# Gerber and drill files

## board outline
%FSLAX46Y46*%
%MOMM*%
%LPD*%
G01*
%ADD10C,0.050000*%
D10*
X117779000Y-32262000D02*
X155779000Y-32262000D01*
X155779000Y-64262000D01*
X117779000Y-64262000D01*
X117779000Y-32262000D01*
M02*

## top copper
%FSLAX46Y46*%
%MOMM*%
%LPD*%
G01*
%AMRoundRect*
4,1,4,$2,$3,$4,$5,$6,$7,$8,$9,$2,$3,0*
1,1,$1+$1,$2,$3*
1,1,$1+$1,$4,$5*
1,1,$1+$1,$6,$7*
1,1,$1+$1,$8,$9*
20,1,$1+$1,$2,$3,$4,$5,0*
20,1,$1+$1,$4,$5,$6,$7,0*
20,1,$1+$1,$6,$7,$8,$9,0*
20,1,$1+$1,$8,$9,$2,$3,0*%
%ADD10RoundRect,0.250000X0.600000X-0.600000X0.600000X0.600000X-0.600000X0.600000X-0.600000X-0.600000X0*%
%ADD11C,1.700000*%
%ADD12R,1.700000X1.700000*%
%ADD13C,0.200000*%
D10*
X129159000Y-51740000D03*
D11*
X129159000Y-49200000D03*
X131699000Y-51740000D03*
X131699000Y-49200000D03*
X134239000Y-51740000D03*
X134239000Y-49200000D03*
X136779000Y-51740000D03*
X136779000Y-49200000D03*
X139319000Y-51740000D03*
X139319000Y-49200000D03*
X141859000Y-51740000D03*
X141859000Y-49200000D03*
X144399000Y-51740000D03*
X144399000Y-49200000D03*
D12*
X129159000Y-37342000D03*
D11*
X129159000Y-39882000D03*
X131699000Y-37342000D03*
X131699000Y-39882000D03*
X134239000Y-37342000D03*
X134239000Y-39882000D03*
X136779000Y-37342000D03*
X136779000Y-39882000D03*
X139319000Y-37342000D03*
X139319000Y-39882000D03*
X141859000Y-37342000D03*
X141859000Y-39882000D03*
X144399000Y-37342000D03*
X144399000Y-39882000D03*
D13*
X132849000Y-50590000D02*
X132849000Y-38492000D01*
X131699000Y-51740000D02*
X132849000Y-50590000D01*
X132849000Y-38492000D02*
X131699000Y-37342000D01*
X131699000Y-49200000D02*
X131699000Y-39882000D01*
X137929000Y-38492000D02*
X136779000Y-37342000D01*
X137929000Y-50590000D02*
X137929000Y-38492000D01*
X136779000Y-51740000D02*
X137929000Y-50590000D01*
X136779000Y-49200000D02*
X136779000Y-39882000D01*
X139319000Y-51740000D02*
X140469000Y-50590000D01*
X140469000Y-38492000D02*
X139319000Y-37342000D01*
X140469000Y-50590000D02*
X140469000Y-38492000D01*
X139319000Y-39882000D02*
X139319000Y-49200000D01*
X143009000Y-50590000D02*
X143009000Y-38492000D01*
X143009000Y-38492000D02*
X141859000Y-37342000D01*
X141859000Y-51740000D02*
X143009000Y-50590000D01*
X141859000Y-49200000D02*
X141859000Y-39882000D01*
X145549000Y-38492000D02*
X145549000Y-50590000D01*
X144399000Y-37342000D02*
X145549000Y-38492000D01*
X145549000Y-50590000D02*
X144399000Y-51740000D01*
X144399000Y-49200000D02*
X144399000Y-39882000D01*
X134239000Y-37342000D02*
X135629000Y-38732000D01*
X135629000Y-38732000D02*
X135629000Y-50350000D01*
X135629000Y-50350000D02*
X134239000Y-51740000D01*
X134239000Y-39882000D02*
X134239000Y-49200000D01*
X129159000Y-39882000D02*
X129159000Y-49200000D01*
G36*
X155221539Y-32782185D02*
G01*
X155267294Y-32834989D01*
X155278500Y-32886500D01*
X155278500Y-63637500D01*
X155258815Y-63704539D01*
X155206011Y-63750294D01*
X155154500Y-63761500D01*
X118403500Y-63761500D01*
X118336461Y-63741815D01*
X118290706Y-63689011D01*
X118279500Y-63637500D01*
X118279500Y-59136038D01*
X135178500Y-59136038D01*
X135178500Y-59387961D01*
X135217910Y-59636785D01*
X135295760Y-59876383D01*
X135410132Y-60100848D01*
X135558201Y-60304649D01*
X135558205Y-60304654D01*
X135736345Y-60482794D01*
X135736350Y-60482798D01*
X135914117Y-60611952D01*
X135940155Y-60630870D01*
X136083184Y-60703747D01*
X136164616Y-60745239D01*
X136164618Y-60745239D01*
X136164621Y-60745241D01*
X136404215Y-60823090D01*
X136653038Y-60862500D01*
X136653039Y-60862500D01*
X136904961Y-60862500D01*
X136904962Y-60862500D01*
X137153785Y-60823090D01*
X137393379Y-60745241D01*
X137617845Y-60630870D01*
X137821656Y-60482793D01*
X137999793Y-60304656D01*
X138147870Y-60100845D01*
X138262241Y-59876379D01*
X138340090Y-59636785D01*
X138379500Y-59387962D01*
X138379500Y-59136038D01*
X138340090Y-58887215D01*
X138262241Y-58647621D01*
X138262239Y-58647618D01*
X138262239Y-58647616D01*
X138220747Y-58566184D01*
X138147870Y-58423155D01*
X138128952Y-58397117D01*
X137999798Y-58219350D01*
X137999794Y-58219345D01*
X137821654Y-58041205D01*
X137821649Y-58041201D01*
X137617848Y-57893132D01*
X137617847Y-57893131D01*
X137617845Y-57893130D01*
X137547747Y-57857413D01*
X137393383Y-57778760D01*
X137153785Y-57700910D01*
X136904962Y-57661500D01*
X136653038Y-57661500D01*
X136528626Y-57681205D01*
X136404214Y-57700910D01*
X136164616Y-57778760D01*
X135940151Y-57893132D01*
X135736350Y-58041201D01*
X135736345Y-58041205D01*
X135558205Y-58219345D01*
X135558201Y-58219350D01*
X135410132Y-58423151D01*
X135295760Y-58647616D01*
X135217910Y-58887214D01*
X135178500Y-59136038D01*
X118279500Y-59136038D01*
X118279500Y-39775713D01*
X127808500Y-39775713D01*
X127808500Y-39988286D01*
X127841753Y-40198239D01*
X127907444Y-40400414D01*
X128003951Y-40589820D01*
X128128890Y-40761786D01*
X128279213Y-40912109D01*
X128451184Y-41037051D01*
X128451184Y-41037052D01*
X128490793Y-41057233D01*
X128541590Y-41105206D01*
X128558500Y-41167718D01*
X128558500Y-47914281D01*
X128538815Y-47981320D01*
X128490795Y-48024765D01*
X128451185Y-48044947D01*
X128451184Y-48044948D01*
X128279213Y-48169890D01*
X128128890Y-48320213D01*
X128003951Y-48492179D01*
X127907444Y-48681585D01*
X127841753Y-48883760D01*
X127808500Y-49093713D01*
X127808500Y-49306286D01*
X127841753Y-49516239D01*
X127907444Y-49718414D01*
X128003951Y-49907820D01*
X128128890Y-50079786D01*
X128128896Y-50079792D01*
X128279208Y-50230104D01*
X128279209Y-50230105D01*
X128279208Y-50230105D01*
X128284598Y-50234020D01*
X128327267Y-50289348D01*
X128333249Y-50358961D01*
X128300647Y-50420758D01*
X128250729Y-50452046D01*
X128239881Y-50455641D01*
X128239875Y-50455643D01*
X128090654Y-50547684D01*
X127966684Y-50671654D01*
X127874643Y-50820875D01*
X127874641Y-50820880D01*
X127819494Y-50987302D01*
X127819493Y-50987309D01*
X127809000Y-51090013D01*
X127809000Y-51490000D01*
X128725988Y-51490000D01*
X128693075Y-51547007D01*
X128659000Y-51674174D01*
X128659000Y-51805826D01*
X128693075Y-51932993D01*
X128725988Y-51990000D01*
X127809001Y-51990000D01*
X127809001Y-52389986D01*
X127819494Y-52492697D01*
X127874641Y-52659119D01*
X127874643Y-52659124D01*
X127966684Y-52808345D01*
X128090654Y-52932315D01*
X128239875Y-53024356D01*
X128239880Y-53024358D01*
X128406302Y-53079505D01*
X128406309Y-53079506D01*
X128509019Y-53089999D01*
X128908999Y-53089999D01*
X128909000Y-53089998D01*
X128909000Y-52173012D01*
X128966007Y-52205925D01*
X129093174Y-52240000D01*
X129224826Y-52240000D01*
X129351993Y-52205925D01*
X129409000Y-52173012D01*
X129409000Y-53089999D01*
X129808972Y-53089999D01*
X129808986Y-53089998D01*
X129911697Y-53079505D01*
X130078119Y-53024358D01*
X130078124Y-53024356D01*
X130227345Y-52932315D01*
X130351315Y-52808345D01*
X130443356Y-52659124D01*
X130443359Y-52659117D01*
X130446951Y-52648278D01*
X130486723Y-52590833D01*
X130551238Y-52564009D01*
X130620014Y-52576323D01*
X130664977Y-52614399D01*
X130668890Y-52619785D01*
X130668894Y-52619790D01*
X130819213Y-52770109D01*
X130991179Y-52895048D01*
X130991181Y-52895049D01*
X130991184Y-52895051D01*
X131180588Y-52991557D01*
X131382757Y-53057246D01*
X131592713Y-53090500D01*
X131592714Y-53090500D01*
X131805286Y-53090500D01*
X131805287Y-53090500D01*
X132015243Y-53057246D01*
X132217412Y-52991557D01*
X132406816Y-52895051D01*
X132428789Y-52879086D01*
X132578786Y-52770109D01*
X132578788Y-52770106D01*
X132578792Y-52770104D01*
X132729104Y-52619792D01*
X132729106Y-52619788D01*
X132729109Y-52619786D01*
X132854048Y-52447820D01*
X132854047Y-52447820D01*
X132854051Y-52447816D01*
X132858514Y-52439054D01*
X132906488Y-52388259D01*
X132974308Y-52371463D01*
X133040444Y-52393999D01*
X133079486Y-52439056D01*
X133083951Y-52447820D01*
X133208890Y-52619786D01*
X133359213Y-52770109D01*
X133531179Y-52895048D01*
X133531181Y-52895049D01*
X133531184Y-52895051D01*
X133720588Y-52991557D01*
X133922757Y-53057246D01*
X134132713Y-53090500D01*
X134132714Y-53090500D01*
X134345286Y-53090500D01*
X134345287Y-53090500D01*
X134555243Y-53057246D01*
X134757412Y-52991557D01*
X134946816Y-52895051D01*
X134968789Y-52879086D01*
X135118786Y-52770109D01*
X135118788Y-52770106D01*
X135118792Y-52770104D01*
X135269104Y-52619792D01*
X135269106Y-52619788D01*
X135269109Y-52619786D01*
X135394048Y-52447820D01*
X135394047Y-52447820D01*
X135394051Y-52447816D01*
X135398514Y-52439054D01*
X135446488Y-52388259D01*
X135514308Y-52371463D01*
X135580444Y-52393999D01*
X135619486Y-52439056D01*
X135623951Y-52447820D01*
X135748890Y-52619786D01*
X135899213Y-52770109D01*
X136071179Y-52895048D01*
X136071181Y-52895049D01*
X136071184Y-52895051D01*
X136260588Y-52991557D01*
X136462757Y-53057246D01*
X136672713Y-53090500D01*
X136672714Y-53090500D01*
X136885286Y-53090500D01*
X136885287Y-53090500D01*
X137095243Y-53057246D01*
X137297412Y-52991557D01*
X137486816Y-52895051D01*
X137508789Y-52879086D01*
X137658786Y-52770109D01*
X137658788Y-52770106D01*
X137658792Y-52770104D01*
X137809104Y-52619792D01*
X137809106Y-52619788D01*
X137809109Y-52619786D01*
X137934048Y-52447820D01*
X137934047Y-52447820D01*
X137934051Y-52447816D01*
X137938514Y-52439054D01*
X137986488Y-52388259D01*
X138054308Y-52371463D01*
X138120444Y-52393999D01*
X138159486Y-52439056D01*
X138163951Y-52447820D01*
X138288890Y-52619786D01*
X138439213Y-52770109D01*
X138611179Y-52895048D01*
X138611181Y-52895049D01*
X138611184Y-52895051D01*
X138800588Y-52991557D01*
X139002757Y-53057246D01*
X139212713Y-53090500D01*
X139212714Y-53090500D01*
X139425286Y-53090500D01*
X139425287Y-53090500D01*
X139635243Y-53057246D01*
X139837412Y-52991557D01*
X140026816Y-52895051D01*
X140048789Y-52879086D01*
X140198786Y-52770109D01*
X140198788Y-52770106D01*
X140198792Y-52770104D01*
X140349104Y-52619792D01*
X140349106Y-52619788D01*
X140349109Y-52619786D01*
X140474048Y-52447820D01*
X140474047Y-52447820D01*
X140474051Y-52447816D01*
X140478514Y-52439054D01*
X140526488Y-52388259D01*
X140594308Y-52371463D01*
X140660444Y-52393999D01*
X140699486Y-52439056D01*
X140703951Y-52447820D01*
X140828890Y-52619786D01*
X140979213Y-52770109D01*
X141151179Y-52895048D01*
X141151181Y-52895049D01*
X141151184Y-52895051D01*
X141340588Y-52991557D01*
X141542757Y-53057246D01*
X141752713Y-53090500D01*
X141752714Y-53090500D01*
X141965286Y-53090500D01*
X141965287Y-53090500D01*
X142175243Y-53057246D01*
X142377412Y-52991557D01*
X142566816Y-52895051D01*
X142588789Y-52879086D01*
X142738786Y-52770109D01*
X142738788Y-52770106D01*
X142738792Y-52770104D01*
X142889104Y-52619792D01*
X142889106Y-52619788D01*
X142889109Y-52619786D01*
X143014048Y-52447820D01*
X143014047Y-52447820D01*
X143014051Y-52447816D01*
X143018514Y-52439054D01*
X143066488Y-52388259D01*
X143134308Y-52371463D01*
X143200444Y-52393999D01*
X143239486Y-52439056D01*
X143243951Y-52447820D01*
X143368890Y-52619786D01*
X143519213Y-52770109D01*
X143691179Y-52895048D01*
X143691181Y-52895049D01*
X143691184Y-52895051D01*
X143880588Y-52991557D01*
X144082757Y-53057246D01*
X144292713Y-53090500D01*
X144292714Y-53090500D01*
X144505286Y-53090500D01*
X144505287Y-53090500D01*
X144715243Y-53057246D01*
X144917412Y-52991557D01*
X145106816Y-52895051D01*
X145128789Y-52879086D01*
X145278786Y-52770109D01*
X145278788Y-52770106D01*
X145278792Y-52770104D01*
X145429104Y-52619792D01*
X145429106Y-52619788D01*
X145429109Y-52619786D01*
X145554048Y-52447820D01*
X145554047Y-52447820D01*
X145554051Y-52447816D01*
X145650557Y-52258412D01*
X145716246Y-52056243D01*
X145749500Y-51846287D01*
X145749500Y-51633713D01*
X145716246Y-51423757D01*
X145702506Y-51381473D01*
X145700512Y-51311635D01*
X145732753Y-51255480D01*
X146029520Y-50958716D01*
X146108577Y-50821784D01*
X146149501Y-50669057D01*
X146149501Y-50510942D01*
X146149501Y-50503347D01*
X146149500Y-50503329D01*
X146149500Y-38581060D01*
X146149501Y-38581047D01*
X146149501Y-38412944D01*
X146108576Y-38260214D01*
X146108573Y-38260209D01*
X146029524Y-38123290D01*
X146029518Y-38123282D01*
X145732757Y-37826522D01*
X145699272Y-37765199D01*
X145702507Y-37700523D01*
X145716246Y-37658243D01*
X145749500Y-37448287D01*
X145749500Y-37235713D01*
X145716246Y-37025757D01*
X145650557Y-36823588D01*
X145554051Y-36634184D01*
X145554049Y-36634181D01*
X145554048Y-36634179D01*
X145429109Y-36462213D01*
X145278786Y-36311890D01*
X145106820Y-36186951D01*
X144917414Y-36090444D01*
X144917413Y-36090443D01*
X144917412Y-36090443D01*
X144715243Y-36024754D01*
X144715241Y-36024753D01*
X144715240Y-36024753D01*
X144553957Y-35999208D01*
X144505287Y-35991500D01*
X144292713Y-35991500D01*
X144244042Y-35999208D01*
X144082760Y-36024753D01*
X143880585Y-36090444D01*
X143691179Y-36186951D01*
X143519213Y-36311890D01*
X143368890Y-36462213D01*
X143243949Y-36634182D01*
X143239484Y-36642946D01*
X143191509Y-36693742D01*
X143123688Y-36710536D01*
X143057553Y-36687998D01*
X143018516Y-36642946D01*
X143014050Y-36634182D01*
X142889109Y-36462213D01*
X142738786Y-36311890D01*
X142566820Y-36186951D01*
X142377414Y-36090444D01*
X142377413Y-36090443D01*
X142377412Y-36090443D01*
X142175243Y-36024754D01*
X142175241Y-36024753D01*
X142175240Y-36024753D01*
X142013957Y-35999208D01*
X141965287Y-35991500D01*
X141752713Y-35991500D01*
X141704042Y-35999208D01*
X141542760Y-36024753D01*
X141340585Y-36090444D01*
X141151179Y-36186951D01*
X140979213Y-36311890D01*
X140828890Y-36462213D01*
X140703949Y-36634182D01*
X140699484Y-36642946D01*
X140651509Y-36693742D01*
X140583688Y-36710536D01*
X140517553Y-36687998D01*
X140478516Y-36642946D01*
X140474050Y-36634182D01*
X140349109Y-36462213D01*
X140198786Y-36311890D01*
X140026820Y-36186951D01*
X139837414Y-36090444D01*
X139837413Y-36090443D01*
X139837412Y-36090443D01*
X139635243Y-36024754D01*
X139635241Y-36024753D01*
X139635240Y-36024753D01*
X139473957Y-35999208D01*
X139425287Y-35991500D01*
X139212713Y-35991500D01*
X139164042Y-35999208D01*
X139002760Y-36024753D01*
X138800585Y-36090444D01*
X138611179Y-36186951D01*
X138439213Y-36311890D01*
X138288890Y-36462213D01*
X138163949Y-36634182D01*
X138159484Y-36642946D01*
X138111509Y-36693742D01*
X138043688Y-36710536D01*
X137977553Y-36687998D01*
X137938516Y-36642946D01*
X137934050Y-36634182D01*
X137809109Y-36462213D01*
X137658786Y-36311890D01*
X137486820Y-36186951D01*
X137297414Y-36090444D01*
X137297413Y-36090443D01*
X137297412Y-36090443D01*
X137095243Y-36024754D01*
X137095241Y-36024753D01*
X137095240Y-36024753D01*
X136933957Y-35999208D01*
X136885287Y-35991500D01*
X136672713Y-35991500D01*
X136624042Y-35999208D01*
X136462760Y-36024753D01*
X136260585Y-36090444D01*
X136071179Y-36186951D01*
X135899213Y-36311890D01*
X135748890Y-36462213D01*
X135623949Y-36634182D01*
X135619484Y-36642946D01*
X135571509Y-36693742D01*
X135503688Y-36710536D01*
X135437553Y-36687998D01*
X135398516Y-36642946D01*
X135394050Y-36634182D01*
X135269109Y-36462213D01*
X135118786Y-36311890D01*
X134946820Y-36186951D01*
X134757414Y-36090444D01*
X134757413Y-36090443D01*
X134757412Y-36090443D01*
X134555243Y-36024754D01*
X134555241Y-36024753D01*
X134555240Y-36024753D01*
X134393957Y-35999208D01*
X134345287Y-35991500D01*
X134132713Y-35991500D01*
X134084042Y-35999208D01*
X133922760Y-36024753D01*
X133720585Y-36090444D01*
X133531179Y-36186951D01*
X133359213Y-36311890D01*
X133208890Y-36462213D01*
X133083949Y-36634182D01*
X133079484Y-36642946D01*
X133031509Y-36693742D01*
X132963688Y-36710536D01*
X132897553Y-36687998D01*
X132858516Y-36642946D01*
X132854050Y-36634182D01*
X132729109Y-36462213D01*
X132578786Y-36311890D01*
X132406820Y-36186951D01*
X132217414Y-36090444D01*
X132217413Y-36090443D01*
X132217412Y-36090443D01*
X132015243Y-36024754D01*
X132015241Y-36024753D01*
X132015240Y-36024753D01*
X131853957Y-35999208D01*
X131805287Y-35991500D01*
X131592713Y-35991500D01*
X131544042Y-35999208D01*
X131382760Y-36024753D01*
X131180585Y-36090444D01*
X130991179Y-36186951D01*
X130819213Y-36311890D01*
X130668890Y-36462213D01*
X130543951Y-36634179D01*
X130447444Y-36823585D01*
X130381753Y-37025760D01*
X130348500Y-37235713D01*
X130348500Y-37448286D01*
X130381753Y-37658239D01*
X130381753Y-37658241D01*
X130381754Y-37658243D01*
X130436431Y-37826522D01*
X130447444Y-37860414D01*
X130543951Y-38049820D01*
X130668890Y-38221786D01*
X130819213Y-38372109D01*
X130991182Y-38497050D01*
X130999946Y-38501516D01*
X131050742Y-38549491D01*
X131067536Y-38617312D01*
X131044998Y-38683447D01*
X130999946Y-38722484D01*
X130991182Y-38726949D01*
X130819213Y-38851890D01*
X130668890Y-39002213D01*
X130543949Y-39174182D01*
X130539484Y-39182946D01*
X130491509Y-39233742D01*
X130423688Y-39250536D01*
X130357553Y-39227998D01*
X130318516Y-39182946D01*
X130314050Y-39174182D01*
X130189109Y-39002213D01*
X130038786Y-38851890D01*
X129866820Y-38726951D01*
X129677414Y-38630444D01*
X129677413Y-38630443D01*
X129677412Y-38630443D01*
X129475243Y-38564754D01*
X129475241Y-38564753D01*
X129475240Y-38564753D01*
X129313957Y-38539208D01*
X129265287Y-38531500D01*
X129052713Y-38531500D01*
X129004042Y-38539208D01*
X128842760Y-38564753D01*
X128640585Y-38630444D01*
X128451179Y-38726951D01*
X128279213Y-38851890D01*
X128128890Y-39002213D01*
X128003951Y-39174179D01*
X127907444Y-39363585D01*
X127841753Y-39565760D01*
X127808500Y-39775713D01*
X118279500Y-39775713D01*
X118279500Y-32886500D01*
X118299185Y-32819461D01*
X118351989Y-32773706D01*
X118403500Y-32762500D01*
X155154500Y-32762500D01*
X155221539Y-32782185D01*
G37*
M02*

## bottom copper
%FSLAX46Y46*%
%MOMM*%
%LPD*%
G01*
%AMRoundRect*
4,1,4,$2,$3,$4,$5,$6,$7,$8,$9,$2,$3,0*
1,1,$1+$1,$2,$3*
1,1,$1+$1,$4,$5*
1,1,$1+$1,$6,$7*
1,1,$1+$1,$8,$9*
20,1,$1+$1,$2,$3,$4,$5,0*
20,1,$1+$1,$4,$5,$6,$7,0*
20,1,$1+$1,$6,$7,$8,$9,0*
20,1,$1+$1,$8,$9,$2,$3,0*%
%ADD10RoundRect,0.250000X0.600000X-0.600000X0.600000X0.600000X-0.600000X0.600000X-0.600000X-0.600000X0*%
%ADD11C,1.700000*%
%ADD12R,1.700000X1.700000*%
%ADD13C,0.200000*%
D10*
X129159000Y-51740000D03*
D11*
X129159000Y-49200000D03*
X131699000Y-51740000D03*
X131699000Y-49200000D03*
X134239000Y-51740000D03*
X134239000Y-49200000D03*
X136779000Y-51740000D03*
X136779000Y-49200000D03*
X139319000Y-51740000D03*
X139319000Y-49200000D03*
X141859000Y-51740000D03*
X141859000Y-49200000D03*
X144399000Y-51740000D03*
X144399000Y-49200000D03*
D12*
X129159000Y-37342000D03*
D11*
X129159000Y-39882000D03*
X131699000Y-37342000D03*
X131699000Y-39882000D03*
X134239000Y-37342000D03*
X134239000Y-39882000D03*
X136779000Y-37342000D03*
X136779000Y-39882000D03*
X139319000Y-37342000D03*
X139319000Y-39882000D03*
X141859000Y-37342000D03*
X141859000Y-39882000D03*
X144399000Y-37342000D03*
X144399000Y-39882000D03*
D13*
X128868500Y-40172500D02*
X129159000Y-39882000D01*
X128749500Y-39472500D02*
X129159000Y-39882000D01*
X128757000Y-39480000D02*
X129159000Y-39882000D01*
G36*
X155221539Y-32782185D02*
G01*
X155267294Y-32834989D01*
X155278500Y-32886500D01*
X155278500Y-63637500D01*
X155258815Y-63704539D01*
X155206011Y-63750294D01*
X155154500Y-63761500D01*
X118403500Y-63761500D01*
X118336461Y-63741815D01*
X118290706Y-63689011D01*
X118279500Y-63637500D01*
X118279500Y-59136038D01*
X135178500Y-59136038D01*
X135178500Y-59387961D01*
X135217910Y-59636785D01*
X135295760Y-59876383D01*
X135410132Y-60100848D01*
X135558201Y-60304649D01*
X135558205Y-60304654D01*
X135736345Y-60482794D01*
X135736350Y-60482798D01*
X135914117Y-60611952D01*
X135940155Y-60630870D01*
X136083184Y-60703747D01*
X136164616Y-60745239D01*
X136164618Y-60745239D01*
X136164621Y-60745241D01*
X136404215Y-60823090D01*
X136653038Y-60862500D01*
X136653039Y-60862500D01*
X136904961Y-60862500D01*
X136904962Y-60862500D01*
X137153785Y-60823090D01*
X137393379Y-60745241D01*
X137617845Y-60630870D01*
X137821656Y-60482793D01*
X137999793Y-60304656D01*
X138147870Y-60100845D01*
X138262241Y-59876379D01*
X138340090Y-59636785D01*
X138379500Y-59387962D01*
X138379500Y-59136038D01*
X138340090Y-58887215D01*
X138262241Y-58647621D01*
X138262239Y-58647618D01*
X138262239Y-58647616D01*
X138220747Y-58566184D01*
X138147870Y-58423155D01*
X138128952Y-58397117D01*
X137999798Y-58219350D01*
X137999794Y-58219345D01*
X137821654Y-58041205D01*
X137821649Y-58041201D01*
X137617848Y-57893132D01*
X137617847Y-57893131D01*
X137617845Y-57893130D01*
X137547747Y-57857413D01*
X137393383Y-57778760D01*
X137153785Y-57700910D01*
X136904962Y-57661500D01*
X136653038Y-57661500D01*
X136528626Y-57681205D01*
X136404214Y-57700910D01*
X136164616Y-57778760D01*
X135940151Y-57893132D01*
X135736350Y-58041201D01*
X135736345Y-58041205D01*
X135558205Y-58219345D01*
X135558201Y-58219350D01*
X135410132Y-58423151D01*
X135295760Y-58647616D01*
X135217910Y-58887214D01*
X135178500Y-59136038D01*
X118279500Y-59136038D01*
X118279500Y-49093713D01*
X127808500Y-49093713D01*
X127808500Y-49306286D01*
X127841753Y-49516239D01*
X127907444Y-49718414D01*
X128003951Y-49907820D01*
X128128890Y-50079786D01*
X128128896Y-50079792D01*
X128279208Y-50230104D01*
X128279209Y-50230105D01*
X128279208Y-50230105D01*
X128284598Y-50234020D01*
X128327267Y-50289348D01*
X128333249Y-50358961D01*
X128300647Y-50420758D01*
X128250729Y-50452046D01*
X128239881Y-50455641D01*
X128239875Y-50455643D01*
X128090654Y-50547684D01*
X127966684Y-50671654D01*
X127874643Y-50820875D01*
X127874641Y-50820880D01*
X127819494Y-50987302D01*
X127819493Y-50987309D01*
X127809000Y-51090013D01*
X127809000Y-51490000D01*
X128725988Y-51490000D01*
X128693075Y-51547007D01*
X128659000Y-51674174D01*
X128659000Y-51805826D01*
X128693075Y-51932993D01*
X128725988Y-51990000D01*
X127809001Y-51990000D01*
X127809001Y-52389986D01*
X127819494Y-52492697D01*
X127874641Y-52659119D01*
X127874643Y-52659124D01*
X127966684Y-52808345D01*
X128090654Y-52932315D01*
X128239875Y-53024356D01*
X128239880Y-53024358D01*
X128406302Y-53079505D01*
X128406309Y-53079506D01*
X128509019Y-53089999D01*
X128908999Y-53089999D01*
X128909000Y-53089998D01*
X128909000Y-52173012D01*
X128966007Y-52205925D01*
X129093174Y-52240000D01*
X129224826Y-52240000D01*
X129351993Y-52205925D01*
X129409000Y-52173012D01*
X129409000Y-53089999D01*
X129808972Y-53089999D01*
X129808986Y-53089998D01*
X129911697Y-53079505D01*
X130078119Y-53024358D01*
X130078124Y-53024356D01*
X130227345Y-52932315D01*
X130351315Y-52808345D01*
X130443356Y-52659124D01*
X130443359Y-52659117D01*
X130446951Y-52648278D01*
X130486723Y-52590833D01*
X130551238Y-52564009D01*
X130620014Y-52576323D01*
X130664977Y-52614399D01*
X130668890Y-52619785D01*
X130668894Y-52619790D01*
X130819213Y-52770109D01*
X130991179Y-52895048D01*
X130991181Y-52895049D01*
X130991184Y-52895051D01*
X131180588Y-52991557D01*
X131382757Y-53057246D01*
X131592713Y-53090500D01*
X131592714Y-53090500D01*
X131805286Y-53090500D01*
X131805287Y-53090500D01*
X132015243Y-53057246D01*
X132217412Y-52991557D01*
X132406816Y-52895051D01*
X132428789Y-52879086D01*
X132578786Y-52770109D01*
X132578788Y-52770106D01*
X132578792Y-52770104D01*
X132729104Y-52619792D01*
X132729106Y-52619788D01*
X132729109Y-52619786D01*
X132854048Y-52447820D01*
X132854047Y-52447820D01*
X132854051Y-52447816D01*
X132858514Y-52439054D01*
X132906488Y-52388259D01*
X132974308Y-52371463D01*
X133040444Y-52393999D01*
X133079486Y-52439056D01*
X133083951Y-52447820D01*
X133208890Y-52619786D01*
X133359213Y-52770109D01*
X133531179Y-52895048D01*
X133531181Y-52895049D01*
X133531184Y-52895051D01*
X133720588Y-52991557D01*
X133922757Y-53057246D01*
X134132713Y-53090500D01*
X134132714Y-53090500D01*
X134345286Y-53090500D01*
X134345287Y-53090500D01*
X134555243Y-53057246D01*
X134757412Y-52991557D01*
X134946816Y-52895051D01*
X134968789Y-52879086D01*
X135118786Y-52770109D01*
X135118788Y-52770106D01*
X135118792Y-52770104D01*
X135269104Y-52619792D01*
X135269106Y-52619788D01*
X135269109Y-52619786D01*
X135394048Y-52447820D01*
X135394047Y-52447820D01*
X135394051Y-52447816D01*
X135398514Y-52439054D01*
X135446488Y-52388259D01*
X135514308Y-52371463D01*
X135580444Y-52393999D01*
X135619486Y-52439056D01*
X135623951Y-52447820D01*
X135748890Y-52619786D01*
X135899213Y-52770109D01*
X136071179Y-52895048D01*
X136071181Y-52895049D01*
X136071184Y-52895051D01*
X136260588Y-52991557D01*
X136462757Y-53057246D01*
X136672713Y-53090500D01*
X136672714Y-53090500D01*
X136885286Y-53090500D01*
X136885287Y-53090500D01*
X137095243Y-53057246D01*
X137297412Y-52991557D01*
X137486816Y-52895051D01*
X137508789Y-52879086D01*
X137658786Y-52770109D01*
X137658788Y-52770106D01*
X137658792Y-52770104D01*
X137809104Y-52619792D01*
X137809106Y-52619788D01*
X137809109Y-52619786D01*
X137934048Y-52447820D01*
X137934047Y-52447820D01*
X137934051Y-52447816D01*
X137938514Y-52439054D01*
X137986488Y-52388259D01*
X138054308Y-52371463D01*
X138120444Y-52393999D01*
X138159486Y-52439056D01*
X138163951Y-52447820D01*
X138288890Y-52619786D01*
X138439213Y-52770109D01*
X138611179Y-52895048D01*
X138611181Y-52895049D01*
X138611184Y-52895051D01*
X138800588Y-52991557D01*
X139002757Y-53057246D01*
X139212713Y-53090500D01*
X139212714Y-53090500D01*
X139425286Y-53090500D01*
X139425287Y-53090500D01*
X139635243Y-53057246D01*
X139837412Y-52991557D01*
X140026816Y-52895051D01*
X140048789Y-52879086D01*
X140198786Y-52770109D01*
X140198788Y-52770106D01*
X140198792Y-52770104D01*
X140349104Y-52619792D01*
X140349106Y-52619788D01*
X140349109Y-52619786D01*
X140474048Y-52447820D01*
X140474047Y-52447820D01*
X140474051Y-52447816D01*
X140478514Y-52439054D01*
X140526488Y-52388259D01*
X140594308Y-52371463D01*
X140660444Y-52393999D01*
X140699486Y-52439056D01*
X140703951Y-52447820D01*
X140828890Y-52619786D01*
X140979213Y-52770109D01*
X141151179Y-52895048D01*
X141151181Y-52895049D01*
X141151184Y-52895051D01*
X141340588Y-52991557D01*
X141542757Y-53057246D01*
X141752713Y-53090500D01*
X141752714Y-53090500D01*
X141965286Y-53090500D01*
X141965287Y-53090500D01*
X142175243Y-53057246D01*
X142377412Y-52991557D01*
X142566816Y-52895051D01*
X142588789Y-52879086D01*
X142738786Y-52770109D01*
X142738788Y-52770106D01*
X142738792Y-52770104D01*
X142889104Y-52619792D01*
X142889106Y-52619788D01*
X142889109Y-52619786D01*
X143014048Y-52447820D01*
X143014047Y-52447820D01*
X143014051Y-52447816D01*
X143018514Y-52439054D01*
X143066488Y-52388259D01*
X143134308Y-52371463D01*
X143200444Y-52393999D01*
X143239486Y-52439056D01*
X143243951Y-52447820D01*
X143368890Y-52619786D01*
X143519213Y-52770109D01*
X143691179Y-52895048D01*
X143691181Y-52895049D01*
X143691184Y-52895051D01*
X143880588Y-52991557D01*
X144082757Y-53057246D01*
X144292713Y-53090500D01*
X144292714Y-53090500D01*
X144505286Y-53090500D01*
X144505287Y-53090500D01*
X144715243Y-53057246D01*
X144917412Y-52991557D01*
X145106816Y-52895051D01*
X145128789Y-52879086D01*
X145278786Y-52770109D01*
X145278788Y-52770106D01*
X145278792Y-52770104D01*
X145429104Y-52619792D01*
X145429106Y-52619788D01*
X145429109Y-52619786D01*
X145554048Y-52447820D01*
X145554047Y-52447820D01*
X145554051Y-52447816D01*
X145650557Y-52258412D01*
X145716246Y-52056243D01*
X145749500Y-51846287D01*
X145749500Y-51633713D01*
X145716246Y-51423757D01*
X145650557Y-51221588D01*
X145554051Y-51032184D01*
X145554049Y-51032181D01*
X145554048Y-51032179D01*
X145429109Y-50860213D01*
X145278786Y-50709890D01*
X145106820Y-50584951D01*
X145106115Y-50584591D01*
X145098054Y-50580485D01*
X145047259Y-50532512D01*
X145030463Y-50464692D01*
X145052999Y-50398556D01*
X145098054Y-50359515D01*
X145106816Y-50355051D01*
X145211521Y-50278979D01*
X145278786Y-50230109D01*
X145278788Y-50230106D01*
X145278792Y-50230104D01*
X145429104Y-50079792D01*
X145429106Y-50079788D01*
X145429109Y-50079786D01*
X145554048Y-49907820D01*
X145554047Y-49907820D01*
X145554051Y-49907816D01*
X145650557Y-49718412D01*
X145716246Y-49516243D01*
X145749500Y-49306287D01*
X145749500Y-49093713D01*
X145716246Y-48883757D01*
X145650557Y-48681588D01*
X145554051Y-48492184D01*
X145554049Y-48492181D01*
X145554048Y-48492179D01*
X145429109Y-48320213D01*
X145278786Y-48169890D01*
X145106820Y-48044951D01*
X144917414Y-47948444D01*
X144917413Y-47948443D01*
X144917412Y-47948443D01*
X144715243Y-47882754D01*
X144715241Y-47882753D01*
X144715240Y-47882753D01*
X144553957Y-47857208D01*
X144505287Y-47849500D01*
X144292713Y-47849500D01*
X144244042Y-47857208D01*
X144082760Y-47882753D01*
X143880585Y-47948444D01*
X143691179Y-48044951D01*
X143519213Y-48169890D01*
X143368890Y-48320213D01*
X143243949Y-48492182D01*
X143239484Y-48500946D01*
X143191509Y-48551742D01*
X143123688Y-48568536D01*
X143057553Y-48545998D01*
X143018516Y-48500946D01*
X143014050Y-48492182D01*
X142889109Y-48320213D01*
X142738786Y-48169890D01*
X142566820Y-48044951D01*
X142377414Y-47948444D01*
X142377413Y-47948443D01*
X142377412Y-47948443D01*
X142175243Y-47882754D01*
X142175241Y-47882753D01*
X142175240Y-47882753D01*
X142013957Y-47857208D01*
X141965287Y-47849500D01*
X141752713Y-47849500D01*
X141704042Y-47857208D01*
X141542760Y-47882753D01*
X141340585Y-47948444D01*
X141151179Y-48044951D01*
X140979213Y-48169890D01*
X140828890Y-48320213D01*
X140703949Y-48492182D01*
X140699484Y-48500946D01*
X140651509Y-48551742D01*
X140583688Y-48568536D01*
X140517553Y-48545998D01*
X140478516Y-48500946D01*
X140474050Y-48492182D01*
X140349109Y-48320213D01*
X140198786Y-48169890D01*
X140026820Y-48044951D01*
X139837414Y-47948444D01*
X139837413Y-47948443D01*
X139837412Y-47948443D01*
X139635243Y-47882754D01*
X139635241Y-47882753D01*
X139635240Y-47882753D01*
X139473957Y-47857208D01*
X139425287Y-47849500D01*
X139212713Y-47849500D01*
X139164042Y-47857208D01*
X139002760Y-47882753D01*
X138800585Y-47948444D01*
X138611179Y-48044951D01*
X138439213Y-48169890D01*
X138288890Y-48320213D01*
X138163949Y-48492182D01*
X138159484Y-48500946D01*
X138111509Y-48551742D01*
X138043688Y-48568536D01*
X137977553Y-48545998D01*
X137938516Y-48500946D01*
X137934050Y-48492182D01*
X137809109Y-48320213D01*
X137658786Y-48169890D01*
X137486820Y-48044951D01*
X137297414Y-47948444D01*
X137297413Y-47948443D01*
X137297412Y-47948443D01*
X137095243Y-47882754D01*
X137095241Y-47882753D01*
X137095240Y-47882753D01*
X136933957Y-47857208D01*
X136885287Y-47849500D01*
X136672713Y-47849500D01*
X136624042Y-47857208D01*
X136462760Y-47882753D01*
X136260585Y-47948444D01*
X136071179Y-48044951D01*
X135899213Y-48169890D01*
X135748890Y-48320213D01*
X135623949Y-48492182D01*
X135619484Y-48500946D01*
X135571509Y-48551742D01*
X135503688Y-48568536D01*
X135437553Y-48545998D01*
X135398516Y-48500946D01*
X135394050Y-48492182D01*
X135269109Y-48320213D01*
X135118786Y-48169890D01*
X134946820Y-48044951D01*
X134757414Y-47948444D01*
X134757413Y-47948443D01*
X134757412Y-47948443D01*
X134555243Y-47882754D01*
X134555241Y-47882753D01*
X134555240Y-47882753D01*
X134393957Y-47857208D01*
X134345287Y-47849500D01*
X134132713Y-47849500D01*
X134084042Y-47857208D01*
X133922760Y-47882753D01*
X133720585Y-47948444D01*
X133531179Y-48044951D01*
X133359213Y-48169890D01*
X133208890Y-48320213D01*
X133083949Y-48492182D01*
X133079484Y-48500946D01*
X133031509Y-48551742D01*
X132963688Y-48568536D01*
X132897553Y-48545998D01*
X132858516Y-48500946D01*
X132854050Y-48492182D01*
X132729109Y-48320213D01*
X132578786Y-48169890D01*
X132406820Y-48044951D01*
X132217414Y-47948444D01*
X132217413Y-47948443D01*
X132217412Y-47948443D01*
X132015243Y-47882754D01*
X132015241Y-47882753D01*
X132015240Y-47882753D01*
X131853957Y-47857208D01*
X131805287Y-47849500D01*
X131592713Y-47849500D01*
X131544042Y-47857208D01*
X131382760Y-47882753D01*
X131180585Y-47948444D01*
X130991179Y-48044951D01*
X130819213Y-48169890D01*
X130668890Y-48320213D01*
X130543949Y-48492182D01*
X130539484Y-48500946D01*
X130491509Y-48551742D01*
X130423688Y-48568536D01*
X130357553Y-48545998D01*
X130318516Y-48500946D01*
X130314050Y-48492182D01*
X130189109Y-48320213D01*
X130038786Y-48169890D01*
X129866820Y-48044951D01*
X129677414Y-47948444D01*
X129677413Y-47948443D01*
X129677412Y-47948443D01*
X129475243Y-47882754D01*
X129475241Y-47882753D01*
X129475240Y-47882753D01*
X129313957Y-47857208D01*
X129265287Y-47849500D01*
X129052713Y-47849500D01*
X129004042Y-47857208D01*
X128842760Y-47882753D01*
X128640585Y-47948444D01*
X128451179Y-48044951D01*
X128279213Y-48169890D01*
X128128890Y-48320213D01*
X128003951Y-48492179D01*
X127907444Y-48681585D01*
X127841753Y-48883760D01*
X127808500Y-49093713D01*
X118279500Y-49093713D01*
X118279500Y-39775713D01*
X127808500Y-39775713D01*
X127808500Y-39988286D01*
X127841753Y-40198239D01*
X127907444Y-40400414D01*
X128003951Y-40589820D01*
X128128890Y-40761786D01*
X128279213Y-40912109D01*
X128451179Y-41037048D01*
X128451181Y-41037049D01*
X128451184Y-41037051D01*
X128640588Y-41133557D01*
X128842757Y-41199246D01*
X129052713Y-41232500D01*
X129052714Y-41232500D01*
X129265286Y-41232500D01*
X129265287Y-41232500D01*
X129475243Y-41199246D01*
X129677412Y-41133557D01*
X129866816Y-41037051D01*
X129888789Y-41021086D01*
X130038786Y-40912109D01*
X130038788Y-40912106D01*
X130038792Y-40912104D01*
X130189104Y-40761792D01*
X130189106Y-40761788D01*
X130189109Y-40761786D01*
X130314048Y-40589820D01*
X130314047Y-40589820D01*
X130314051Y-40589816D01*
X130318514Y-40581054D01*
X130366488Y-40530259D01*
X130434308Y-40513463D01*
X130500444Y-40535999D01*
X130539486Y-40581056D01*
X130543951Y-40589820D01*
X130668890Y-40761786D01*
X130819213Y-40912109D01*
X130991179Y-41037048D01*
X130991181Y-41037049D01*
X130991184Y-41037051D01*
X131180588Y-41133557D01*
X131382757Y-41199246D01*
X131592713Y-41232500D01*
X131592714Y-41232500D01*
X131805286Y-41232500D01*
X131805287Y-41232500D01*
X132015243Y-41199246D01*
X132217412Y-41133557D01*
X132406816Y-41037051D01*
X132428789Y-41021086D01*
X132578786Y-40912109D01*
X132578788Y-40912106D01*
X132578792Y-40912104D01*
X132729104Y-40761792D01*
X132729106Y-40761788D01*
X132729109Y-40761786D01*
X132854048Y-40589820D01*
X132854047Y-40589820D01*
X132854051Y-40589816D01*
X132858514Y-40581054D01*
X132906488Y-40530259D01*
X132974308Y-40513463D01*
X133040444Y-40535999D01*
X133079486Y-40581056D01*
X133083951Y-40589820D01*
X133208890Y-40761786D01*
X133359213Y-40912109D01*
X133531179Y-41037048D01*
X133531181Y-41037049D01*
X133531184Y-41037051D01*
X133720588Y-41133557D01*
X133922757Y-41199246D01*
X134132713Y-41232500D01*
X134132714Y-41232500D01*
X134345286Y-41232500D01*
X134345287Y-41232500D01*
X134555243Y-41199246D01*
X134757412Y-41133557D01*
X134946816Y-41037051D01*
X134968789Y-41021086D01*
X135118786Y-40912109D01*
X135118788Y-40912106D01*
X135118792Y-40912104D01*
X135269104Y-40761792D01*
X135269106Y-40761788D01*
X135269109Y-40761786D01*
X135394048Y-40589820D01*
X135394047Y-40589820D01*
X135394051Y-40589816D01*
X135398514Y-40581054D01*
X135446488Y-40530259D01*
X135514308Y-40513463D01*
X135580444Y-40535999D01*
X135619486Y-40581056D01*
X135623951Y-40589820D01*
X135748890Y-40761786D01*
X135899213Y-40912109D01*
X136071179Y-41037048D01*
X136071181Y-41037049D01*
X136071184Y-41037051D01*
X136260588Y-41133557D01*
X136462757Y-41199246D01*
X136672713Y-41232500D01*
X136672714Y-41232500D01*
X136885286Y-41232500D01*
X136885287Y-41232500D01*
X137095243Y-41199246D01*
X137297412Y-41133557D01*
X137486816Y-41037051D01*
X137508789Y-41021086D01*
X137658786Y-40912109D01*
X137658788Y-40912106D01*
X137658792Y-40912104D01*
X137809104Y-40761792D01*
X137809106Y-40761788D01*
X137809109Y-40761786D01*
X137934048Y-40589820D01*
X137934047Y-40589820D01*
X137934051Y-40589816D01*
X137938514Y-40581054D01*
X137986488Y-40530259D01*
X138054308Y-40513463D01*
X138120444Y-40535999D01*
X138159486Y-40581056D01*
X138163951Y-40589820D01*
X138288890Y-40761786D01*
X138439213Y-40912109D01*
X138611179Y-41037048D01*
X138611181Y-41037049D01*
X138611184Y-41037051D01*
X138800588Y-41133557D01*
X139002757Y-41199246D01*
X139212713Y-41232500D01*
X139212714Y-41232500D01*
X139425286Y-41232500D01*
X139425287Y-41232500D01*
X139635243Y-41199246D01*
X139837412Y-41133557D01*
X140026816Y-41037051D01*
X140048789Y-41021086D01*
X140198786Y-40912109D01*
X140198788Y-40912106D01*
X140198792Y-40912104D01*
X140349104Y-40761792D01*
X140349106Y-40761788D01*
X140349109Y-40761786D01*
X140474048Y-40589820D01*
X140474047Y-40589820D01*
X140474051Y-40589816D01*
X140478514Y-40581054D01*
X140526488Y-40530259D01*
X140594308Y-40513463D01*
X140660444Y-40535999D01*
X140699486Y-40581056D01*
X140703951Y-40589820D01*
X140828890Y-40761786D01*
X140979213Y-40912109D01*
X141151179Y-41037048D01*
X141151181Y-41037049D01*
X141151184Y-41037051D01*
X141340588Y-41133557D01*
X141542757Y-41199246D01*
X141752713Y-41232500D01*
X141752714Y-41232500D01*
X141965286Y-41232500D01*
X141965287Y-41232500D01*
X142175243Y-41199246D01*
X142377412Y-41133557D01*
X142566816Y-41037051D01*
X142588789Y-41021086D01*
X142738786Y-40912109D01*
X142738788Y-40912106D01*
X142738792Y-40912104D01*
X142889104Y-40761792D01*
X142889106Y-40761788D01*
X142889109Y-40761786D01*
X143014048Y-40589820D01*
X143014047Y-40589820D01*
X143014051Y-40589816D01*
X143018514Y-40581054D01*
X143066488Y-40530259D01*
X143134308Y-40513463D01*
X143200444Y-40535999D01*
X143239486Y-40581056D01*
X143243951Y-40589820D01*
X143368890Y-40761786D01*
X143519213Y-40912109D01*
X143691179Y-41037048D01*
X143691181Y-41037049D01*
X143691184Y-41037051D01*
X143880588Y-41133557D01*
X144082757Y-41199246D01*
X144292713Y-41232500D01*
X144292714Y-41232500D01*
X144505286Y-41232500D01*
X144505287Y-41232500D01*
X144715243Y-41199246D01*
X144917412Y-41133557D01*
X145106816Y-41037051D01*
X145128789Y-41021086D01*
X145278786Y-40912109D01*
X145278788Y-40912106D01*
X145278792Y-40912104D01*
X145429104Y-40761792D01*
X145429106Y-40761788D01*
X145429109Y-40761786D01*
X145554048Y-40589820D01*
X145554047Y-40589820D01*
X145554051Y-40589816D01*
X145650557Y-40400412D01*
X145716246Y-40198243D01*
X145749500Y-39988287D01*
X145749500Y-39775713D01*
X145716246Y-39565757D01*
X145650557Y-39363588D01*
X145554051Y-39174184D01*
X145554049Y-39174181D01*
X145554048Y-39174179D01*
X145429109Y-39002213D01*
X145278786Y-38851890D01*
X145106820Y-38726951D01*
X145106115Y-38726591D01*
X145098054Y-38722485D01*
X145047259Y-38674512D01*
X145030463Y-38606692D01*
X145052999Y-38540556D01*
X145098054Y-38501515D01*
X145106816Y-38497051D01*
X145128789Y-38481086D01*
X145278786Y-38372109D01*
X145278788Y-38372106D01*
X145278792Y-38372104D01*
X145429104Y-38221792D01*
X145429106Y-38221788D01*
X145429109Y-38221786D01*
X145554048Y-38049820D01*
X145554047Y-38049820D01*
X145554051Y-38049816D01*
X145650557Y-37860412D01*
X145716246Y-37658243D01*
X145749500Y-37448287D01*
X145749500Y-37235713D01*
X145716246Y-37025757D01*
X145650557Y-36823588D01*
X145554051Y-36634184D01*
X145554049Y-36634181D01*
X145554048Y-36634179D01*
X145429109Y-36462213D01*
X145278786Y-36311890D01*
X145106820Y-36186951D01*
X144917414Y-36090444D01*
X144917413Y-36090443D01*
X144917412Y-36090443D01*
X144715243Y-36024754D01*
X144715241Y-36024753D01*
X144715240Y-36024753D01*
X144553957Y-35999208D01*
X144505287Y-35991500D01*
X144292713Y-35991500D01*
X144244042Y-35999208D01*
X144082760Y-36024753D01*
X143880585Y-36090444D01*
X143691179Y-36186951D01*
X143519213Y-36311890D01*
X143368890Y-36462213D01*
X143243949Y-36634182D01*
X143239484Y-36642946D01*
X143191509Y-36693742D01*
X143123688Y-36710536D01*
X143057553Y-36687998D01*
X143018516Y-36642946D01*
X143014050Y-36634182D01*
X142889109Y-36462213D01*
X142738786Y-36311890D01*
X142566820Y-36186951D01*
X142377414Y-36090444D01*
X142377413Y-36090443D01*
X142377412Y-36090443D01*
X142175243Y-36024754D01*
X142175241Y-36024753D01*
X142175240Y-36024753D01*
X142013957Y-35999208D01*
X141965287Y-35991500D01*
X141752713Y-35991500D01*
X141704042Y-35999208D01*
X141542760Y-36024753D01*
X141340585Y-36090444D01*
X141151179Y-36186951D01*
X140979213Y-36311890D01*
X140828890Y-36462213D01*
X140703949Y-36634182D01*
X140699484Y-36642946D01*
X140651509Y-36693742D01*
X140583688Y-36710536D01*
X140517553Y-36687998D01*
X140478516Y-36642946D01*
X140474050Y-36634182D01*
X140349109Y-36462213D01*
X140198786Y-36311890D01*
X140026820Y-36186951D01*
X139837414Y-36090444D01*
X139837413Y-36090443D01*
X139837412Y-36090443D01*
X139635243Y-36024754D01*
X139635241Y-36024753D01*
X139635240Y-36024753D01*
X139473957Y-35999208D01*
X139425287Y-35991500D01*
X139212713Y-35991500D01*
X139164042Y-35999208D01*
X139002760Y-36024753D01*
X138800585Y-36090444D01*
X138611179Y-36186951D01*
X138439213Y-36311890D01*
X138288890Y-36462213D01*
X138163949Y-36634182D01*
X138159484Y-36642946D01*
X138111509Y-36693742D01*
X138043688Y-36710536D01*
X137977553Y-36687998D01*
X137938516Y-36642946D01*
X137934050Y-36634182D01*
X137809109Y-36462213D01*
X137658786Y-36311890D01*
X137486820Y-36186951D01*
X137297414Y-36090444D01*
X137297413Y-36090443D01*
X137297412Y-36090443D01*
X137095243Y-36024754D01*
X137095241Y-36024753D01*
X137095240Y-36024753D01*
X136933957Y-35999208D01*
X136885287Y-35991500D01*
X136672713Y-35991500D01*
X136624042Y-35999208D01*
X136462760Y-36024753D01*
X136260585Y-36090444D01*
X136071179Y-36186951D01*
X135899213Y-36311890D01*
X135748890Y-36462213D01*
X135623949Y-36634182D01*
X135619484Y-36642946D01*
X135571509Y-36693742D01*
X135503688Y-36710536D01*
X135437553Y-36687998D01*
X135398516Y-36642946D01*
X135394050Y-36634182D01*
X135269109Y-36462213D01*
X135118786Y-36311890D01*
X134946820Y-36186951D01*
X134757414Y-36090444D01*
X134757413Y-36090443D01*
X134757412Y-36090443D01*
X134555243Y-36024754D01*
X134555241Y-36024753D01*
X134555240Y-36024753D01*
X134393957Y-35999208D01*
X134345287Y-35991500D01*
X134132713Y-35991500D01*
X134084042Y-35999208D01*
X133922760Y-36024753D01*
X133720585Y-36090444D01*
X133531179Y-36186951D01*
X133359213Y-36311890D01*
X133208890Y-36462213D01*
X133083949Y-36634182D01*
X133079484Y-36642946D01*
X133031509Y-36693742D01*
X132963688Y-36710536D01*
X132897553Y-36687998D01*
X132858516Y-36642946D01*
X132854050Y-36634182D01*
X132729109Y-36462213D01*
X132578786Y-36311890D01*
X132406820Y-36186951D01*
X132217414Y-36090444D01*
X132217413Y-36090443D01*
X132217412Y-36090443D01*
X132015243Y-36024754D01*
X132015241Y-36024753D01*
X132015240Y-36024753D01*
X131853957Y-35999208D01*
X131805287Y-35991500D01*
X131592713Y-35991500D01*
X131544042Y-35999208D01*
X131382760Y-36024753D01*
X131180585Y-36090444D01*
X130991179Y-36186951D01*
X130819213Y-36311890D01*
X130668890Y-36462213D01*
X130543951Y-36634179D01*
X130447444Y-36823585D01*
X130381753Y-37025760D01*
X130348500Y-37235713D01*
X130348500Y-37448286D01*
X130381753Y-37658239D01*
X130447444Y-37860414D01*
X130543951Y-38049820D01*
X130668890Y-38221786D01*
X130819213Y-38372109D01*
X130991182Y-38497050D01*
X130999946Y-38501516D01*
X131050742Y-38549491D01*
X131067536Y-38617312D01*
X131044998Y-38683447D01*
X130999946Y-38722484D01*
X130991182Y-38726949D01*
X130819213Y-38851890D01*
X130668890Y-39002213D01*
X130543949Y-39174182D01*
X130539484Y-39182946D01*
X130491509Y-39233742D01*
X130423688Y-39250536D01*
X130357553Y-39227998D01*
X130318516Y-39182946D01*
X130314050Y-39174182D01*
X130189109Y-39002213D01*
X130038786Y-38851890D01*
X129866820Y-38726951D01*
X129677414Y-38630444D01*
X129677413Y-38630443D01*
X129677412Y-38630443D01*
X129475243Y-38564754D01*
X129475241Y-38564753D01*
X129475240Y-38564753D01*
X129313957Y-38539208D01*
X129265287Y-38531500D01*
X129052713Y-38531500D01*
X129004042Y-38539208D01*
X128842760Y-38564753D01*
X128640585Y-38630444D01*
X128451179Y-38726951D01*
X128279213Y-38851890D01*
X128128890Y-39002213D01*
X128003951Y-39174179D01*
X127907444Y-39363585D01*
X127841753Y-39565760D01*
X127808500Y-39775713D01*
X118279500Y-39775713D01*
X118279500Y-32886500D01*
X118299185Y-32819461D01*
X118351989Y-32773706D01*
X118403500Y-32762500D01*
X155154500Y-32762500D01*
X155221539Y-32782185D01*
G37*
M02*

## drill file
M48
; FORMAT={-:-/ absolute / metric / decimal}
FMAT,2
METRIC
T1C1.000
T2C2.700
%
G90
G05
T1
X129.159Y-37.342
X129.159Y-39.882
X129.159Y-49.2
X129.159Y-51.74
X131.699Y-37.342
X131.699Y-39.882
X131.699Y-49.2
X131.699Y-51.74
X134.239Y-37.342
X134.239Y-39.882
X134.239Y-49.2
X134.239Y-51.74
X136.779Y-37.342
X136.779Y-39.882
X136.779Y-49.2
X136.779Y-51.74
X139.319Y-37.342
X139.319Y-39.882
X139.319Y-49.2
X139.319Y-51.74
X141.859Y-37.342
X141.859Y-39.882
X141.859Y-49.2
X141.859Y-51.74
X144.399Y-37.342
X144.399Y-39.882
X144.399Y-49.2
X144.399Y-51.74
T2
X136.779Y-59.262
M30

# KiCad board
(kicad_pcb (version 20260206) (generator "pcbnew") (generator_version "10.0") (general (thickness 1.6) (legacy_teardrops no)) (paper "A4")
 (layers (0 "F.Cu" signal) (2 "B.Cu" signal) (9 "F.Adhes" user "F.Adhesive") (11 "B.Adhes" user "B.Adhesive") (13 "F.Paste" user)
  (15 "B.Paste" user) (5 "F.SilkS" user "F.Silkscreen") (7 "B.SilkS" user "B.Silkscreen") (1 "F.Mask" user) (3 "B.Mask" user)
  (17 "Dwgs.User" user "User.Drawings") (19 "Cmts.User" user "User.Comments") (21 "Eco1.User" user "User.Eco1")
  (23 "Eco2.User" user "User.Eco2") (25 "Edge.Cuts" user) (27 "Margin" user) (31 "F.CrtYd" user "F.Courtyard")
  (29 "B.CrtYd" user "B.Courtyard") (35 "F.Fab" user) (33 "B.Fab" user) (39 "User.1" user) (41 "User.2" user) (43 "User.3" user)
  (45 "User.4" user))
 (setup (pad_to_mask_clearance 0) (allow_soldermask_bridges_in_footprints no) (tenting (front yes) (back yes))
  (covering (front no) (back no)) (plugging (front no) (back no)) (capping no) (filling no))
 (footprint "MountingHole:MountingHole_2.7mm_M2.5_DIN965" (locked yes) (layer "F.Cu") (at 136.779 59.262)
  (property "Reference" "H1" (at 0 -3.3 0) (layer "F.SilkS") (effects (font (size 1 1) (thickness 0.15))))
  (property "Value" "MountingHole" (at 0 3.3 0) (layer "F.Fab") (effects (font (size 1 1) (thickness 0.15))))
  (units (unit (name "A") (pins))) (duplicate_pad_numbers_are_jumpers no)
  (pad "" np_thru_hole circle (at 0 0) (size 2.7 2.7) (drill 2.7) (layers "*.Cu" "*.Mask")))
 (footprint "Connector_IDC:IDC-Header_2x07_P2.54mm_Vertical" (layer "F.Cu") (at 129.159 51.74 90)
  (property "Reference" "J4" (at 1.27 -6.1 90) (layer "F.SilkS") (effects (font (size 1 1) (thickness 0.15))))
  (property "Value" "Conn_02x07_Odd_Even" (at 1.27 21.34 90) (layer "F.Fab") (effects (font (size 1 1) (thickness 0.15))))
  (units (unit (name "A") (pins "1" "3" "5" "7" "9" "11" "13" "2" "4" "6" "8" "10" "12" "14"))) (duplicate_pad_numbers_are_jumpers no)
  (pad "1" thru_hole roundrect (at 0 0 90) (size 1.7 1.7) (drill 1) (layers "*.Cu" "*.Mask") (remove_unused_layers no)
   (roundrect_rratio 0.147059) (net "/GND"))
  (pad "2" thru_hole circle (at 2.54 0 90) (size 1.7 1.7) (drill 1) (layers "*.Cu" "*.Mask") (remove_unused_layers no) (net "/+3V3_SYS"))
  (pad "3" thru_hole circle (at 0 2.54 90) (size 1.7 1.7) (drill 1) (layers "*.Cu" "*.Mask") (remove_unused_layers no) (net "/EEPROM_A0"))
  (pad "4" thru_hole circle (at 2.54 2.54 90) (size 1.7 1.7) (drill 1) (layers "*.Cu" "*.Mask") (remove_unused_layers no) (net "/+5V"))
  (pad "5" thru_hole circle (at 0 5.08 90) (size 1.7 1.7) (drill 1) (layers "*.Cu" "*.Mask") (remove_unused_layers no) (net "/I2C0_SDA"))
  (pad "6" thru_hole circle (at 2.54 5.08 90) (size 1.7 1.7) (drill 1) (layers "*.Cu" "*.Mask") (remove_unused_layers no) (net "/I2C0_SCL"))
  (pad "7" thru_hole circle (at 0 7.62 90) (size 1.7 1.7) (drill 1) (layers "*.Cu" "*.Mask") (remove_unused_layers no) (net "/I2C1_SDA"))
  (pad "8" thru_hole circle (at 2.54 7.62 90) (size 1.7 1.7) (drill 1) (layers "*.Cu" "*.Mask") (remove_unused_layers no) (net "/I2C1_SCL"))
  (pad "9" thru_hole circle (at 0 10.16 90) (size 1.7 1.7) (drill 1) (layers "*.Cu" "*.Mask") (remove_unused_layers no) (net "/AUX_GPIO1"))
  (pad "10" thru_hole circle (at 2.54 10.16 90) (size 1.7 1.7) (drill 1) (layers "*.Cu" "*.Mask") (remove_unused_layers no)
   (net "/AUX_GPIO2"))
  (pad "11" thru_hole circle (at 0 12.7 90) (size 1.7 1.7) (drill 1) (layers "*.Cu" "*.Mask") (remove_unused_layers no) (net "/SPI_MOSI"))
  (pad "12" thru_hole circle (at 2.54 12.7 90) (size 1.7 1.7) (drill 1) (layers "*.Cu" "*.Mask") (remove_unused_layers no) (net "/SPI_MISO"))
  (pad "13" thru_hole circle (at 0 15.24 90) (size 1.7 1.7) (drill 1) (layers "*.Cu" "*.Mask") (remove_unused_layers no) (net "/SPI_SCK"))
  (pad "14" thru_hole circle (at 2.54 15.24 90) (size 1.7 1.7) (drill 1) (layers "*.Cu" "*.Mask") (remove_unused_layers no) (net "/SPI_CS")))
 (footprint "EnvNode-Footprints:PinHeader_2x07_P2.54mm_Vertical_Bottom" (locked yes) (layer "B.Cu") (at 129.159 37.342 -90)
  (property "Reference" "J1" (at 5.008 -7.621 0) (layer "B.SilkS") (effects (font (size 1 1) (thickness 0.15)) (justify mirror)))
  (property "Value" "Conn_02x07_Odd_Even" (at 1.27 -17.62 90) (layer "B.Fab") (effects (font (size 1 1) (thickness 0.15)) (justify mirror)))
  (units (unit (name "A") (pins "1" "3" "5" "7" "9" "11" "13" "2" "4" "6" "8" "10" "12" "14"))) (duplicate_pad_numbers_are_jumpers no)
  (pad "1" thru_hole rect (at 0 0 270) (size 1.7 1.7) (drill 1) (layers "*.Cu" "*.Mask") (remove_unused_layers no) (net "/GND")
   (zone_connect 2))
  (pad "2" thru_hole circle (at 2.54 0 270) (size 1.7 1.7) (drill 1) (layers "*.Cu" "*.Mask") (remove_unused_layers no) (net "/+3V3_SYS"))
  (pad "3" thru_hole circle (at 0 -2.54 270) (size 1.7 1.7) (drill 1) (layers "*.Cu" "*.Mask") (remove_unused_layers no) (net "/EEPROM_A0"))
  (pad "4" thru_hole circle (at 2.54 -2.54 270) (size 1.7 1.7) (drill 1) (layers "*.Cu" "*.Mask") (remove_unused_layers no) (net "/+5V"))
  (pad "5" thru_hole circle (at 0 -5.08 270) (size 1.7 1.7) (drill 1) (layers "*.Cu" "*.Mask") (remove_unused_layers no) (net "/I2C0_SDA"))
  (pad "6" thru_hole circle (at 2.54 -5.08 270) (size 1.7 1.7) (drill 1) (layers "*.Cu" "*.Mask") (remove_unused_layers no)
   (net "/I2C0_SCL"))
  (pad "7" thru_hole circle (at 0 -7.62 270) (size 1.7 1.7) (drill 1) (layers "*.Cu" "*.Mask") (remove_unused_layers no) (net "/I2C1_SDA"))
  (pad "8" thru_hole circle (at 2.54 -7.62 270) (size 1.7 1.7) (drill 1) (layers "*.Cu" "*.Mask") (remove_unused_layers no)
   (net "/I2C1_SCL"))
  (pad "9" thru_hole circle (at 0 -10.16 270) (size 1.7 1.7) (drill 1) (layers "*.Cu" "*.Mask") (remove_unused_layers no) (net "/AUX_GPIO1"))
  (pad "10" thru_hole circle (at 2.54 -10.16 270) (size 1.7 1.7) (drill 1) (layers "*.Cu" "*.Mask") (remove_unused_layers no)
   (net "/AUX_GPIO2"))
  (pad "11" thru_hole circle (at 0 -12.7 270) (size 1.7 1.7) (drill 1) (layers "*.Cu" "*.Mask") (remove_unused_layers no) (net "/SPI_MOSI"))
  (pad "12" thru_hole circle (at 2.54 -12.7 270) (size 1.7 1.7) (drill 1) (layers "*.Cu" "*.Mask") (remove_unused_layers no)
   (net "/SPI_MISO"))
  (pad "13" thru_hole circle (at 0 -15.24 270) (size 1.7 1.7) (drill 1) (layers "*.Cu" "*.Mask") (remove_unused_layers no) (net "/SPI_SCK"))
  (pad "14" thru_hole circle (at 2.54 -15.24 270) (size 1.7 1.7) (drill 1) (layers "*.Cu" "*.Mask") (remove_unused_layers no)
   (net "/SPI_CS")))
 (gr_rect (start 117.779 32.262) (end 155.779 64.262) (stroke (width 0.05) (type solid)) (fill no) (locked yes) (layer "Edge.Cuts"))
 (segment (start 132.849 50.59) (end 132.849 38.492) (width 0.2) (layer "F.Cu") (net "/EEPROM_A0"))
 (segment (start 131.699 51.74) (end 132.849 50.59) (width 0.2) (layer "F.Cu") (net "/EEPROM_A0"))
 (segment (start 132.849 38.492) (end 131.699 37.342) (width 0.2) (layer "F.Cu") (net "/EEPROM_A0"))
 (segment (start 131.699 49.2) (end 131.699 39.882) (width 0.2) (layer "F.Cu") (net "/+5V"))
 (segment (start 137.929 38.492) (end 136.779 37.342) (width 0.2) (layer "F.Cu") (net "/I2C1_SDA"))
 (segment (start 137.929 50.59) (end 137.929 38.492) (width 0.2) (layer "F.Cu") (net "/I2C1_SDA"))
 (segment (start 136.779 51.74) (end 137.929 50.59) (width 0.2) (layer "F.Cu") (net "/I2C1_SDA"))
 (segment (start 136.779 49.2) (end 136.779 39.882) (width 0.2) (layer "F.Cu") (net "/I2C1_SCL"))
 (segment (start 139.319 51.74) (end 140.469 50.59) (width 0.2) (layer "F.Cu") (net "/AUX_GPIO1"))
 (segment (start 140.469 38.492) (end 139.319 37.342) (width 0.2) (layer "F.Cu") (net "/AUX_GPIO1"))
 (segment (start 140.469 50.59) (end 140.469 38.492) (width 0.2) (layer "F.Cu") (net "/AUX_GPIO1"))
 (segment (start 139.319 39.882) (end 139.319 49.2) (width 0.2) (layer "F.Cu") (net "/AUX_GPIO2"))
 (segment (start 143.009 50.59) (end 143.009 38.492) (width 0.2) (layer "F.Cu") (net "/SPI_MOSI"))
 (segment (start 143.009 38.492) (end 141.859 37.342) (width 0.2) (layer "F.Cu") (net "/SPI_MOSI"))
 (segment (start 141.859 51.74) (end 143.009 50.59) (width 0.2) (layer "F.Cu") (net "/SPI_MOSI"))
 (segment (start 141.859 49.2) (end 141.859 39.882) (width 0.2) (layer "F.Cu") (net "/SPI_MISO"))
 (segment (start 145.549 38.492) (end 145.549 50.59) (width 0.2) (layer "F.Cu") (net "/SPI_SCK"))
 (segment (start 144.399 37.342) (end 145.549 38.492) (width 0.2) (layer "F.Cu") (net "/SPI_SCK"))
 (segment (start 145.549 50.59) (end 144.399 51.74) (width 0.2) (layer "F.Cu") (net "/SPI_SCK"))
 (segment (start 144.399 49.2) (end 144.399 39.882) (width 0.2) (layer "F.Cu") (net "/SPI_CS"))
 (segment (start 134.239 37.342) (end 135.629 38.732) (width 0.2) (layer "F.Cu") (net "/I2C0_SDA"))
 (segment (start 135.629 38.732) (end 135.629 50.35) (width 0.2) (layer "F.Cu") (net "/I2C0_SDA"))
 (segment (start 135.629 50.35) (end 134.239 51.74) (width 0.2) (layer "F.Cu") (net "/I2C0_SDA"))
 (segment (start 134.239 39.882) (end 134.239 49.2) (width 0.2) (layer "F.Cu") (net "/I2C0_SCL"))
 (segment (start 129.159 39.882) (end 129.159 49.2) (width 0.2) (layer "F.Cu") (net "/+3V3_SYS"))
 (segment (start 128.8685 40.1725) (end 129.159 39.882) (width 0.2) (layer "B.Cu") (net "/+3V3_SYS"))
 (segment (start 128.7495 39.4725) (end 129.159 39.882) (width 0.2) (layer "B.Cu") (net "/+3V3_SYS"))
 (segment (start 128.757 39.48) (end 129.159 39.882) (width 0.2) (layer "B.Cu") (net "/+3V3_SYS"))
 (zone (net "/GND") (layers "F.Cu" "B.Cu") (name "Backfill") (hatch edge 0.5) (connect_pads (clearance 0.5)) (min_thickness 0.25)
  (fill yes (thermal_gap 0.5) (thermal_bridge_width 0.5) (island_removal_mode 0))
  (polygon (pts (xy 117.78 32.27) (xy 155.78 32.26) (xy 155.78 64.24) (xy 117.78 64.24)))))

